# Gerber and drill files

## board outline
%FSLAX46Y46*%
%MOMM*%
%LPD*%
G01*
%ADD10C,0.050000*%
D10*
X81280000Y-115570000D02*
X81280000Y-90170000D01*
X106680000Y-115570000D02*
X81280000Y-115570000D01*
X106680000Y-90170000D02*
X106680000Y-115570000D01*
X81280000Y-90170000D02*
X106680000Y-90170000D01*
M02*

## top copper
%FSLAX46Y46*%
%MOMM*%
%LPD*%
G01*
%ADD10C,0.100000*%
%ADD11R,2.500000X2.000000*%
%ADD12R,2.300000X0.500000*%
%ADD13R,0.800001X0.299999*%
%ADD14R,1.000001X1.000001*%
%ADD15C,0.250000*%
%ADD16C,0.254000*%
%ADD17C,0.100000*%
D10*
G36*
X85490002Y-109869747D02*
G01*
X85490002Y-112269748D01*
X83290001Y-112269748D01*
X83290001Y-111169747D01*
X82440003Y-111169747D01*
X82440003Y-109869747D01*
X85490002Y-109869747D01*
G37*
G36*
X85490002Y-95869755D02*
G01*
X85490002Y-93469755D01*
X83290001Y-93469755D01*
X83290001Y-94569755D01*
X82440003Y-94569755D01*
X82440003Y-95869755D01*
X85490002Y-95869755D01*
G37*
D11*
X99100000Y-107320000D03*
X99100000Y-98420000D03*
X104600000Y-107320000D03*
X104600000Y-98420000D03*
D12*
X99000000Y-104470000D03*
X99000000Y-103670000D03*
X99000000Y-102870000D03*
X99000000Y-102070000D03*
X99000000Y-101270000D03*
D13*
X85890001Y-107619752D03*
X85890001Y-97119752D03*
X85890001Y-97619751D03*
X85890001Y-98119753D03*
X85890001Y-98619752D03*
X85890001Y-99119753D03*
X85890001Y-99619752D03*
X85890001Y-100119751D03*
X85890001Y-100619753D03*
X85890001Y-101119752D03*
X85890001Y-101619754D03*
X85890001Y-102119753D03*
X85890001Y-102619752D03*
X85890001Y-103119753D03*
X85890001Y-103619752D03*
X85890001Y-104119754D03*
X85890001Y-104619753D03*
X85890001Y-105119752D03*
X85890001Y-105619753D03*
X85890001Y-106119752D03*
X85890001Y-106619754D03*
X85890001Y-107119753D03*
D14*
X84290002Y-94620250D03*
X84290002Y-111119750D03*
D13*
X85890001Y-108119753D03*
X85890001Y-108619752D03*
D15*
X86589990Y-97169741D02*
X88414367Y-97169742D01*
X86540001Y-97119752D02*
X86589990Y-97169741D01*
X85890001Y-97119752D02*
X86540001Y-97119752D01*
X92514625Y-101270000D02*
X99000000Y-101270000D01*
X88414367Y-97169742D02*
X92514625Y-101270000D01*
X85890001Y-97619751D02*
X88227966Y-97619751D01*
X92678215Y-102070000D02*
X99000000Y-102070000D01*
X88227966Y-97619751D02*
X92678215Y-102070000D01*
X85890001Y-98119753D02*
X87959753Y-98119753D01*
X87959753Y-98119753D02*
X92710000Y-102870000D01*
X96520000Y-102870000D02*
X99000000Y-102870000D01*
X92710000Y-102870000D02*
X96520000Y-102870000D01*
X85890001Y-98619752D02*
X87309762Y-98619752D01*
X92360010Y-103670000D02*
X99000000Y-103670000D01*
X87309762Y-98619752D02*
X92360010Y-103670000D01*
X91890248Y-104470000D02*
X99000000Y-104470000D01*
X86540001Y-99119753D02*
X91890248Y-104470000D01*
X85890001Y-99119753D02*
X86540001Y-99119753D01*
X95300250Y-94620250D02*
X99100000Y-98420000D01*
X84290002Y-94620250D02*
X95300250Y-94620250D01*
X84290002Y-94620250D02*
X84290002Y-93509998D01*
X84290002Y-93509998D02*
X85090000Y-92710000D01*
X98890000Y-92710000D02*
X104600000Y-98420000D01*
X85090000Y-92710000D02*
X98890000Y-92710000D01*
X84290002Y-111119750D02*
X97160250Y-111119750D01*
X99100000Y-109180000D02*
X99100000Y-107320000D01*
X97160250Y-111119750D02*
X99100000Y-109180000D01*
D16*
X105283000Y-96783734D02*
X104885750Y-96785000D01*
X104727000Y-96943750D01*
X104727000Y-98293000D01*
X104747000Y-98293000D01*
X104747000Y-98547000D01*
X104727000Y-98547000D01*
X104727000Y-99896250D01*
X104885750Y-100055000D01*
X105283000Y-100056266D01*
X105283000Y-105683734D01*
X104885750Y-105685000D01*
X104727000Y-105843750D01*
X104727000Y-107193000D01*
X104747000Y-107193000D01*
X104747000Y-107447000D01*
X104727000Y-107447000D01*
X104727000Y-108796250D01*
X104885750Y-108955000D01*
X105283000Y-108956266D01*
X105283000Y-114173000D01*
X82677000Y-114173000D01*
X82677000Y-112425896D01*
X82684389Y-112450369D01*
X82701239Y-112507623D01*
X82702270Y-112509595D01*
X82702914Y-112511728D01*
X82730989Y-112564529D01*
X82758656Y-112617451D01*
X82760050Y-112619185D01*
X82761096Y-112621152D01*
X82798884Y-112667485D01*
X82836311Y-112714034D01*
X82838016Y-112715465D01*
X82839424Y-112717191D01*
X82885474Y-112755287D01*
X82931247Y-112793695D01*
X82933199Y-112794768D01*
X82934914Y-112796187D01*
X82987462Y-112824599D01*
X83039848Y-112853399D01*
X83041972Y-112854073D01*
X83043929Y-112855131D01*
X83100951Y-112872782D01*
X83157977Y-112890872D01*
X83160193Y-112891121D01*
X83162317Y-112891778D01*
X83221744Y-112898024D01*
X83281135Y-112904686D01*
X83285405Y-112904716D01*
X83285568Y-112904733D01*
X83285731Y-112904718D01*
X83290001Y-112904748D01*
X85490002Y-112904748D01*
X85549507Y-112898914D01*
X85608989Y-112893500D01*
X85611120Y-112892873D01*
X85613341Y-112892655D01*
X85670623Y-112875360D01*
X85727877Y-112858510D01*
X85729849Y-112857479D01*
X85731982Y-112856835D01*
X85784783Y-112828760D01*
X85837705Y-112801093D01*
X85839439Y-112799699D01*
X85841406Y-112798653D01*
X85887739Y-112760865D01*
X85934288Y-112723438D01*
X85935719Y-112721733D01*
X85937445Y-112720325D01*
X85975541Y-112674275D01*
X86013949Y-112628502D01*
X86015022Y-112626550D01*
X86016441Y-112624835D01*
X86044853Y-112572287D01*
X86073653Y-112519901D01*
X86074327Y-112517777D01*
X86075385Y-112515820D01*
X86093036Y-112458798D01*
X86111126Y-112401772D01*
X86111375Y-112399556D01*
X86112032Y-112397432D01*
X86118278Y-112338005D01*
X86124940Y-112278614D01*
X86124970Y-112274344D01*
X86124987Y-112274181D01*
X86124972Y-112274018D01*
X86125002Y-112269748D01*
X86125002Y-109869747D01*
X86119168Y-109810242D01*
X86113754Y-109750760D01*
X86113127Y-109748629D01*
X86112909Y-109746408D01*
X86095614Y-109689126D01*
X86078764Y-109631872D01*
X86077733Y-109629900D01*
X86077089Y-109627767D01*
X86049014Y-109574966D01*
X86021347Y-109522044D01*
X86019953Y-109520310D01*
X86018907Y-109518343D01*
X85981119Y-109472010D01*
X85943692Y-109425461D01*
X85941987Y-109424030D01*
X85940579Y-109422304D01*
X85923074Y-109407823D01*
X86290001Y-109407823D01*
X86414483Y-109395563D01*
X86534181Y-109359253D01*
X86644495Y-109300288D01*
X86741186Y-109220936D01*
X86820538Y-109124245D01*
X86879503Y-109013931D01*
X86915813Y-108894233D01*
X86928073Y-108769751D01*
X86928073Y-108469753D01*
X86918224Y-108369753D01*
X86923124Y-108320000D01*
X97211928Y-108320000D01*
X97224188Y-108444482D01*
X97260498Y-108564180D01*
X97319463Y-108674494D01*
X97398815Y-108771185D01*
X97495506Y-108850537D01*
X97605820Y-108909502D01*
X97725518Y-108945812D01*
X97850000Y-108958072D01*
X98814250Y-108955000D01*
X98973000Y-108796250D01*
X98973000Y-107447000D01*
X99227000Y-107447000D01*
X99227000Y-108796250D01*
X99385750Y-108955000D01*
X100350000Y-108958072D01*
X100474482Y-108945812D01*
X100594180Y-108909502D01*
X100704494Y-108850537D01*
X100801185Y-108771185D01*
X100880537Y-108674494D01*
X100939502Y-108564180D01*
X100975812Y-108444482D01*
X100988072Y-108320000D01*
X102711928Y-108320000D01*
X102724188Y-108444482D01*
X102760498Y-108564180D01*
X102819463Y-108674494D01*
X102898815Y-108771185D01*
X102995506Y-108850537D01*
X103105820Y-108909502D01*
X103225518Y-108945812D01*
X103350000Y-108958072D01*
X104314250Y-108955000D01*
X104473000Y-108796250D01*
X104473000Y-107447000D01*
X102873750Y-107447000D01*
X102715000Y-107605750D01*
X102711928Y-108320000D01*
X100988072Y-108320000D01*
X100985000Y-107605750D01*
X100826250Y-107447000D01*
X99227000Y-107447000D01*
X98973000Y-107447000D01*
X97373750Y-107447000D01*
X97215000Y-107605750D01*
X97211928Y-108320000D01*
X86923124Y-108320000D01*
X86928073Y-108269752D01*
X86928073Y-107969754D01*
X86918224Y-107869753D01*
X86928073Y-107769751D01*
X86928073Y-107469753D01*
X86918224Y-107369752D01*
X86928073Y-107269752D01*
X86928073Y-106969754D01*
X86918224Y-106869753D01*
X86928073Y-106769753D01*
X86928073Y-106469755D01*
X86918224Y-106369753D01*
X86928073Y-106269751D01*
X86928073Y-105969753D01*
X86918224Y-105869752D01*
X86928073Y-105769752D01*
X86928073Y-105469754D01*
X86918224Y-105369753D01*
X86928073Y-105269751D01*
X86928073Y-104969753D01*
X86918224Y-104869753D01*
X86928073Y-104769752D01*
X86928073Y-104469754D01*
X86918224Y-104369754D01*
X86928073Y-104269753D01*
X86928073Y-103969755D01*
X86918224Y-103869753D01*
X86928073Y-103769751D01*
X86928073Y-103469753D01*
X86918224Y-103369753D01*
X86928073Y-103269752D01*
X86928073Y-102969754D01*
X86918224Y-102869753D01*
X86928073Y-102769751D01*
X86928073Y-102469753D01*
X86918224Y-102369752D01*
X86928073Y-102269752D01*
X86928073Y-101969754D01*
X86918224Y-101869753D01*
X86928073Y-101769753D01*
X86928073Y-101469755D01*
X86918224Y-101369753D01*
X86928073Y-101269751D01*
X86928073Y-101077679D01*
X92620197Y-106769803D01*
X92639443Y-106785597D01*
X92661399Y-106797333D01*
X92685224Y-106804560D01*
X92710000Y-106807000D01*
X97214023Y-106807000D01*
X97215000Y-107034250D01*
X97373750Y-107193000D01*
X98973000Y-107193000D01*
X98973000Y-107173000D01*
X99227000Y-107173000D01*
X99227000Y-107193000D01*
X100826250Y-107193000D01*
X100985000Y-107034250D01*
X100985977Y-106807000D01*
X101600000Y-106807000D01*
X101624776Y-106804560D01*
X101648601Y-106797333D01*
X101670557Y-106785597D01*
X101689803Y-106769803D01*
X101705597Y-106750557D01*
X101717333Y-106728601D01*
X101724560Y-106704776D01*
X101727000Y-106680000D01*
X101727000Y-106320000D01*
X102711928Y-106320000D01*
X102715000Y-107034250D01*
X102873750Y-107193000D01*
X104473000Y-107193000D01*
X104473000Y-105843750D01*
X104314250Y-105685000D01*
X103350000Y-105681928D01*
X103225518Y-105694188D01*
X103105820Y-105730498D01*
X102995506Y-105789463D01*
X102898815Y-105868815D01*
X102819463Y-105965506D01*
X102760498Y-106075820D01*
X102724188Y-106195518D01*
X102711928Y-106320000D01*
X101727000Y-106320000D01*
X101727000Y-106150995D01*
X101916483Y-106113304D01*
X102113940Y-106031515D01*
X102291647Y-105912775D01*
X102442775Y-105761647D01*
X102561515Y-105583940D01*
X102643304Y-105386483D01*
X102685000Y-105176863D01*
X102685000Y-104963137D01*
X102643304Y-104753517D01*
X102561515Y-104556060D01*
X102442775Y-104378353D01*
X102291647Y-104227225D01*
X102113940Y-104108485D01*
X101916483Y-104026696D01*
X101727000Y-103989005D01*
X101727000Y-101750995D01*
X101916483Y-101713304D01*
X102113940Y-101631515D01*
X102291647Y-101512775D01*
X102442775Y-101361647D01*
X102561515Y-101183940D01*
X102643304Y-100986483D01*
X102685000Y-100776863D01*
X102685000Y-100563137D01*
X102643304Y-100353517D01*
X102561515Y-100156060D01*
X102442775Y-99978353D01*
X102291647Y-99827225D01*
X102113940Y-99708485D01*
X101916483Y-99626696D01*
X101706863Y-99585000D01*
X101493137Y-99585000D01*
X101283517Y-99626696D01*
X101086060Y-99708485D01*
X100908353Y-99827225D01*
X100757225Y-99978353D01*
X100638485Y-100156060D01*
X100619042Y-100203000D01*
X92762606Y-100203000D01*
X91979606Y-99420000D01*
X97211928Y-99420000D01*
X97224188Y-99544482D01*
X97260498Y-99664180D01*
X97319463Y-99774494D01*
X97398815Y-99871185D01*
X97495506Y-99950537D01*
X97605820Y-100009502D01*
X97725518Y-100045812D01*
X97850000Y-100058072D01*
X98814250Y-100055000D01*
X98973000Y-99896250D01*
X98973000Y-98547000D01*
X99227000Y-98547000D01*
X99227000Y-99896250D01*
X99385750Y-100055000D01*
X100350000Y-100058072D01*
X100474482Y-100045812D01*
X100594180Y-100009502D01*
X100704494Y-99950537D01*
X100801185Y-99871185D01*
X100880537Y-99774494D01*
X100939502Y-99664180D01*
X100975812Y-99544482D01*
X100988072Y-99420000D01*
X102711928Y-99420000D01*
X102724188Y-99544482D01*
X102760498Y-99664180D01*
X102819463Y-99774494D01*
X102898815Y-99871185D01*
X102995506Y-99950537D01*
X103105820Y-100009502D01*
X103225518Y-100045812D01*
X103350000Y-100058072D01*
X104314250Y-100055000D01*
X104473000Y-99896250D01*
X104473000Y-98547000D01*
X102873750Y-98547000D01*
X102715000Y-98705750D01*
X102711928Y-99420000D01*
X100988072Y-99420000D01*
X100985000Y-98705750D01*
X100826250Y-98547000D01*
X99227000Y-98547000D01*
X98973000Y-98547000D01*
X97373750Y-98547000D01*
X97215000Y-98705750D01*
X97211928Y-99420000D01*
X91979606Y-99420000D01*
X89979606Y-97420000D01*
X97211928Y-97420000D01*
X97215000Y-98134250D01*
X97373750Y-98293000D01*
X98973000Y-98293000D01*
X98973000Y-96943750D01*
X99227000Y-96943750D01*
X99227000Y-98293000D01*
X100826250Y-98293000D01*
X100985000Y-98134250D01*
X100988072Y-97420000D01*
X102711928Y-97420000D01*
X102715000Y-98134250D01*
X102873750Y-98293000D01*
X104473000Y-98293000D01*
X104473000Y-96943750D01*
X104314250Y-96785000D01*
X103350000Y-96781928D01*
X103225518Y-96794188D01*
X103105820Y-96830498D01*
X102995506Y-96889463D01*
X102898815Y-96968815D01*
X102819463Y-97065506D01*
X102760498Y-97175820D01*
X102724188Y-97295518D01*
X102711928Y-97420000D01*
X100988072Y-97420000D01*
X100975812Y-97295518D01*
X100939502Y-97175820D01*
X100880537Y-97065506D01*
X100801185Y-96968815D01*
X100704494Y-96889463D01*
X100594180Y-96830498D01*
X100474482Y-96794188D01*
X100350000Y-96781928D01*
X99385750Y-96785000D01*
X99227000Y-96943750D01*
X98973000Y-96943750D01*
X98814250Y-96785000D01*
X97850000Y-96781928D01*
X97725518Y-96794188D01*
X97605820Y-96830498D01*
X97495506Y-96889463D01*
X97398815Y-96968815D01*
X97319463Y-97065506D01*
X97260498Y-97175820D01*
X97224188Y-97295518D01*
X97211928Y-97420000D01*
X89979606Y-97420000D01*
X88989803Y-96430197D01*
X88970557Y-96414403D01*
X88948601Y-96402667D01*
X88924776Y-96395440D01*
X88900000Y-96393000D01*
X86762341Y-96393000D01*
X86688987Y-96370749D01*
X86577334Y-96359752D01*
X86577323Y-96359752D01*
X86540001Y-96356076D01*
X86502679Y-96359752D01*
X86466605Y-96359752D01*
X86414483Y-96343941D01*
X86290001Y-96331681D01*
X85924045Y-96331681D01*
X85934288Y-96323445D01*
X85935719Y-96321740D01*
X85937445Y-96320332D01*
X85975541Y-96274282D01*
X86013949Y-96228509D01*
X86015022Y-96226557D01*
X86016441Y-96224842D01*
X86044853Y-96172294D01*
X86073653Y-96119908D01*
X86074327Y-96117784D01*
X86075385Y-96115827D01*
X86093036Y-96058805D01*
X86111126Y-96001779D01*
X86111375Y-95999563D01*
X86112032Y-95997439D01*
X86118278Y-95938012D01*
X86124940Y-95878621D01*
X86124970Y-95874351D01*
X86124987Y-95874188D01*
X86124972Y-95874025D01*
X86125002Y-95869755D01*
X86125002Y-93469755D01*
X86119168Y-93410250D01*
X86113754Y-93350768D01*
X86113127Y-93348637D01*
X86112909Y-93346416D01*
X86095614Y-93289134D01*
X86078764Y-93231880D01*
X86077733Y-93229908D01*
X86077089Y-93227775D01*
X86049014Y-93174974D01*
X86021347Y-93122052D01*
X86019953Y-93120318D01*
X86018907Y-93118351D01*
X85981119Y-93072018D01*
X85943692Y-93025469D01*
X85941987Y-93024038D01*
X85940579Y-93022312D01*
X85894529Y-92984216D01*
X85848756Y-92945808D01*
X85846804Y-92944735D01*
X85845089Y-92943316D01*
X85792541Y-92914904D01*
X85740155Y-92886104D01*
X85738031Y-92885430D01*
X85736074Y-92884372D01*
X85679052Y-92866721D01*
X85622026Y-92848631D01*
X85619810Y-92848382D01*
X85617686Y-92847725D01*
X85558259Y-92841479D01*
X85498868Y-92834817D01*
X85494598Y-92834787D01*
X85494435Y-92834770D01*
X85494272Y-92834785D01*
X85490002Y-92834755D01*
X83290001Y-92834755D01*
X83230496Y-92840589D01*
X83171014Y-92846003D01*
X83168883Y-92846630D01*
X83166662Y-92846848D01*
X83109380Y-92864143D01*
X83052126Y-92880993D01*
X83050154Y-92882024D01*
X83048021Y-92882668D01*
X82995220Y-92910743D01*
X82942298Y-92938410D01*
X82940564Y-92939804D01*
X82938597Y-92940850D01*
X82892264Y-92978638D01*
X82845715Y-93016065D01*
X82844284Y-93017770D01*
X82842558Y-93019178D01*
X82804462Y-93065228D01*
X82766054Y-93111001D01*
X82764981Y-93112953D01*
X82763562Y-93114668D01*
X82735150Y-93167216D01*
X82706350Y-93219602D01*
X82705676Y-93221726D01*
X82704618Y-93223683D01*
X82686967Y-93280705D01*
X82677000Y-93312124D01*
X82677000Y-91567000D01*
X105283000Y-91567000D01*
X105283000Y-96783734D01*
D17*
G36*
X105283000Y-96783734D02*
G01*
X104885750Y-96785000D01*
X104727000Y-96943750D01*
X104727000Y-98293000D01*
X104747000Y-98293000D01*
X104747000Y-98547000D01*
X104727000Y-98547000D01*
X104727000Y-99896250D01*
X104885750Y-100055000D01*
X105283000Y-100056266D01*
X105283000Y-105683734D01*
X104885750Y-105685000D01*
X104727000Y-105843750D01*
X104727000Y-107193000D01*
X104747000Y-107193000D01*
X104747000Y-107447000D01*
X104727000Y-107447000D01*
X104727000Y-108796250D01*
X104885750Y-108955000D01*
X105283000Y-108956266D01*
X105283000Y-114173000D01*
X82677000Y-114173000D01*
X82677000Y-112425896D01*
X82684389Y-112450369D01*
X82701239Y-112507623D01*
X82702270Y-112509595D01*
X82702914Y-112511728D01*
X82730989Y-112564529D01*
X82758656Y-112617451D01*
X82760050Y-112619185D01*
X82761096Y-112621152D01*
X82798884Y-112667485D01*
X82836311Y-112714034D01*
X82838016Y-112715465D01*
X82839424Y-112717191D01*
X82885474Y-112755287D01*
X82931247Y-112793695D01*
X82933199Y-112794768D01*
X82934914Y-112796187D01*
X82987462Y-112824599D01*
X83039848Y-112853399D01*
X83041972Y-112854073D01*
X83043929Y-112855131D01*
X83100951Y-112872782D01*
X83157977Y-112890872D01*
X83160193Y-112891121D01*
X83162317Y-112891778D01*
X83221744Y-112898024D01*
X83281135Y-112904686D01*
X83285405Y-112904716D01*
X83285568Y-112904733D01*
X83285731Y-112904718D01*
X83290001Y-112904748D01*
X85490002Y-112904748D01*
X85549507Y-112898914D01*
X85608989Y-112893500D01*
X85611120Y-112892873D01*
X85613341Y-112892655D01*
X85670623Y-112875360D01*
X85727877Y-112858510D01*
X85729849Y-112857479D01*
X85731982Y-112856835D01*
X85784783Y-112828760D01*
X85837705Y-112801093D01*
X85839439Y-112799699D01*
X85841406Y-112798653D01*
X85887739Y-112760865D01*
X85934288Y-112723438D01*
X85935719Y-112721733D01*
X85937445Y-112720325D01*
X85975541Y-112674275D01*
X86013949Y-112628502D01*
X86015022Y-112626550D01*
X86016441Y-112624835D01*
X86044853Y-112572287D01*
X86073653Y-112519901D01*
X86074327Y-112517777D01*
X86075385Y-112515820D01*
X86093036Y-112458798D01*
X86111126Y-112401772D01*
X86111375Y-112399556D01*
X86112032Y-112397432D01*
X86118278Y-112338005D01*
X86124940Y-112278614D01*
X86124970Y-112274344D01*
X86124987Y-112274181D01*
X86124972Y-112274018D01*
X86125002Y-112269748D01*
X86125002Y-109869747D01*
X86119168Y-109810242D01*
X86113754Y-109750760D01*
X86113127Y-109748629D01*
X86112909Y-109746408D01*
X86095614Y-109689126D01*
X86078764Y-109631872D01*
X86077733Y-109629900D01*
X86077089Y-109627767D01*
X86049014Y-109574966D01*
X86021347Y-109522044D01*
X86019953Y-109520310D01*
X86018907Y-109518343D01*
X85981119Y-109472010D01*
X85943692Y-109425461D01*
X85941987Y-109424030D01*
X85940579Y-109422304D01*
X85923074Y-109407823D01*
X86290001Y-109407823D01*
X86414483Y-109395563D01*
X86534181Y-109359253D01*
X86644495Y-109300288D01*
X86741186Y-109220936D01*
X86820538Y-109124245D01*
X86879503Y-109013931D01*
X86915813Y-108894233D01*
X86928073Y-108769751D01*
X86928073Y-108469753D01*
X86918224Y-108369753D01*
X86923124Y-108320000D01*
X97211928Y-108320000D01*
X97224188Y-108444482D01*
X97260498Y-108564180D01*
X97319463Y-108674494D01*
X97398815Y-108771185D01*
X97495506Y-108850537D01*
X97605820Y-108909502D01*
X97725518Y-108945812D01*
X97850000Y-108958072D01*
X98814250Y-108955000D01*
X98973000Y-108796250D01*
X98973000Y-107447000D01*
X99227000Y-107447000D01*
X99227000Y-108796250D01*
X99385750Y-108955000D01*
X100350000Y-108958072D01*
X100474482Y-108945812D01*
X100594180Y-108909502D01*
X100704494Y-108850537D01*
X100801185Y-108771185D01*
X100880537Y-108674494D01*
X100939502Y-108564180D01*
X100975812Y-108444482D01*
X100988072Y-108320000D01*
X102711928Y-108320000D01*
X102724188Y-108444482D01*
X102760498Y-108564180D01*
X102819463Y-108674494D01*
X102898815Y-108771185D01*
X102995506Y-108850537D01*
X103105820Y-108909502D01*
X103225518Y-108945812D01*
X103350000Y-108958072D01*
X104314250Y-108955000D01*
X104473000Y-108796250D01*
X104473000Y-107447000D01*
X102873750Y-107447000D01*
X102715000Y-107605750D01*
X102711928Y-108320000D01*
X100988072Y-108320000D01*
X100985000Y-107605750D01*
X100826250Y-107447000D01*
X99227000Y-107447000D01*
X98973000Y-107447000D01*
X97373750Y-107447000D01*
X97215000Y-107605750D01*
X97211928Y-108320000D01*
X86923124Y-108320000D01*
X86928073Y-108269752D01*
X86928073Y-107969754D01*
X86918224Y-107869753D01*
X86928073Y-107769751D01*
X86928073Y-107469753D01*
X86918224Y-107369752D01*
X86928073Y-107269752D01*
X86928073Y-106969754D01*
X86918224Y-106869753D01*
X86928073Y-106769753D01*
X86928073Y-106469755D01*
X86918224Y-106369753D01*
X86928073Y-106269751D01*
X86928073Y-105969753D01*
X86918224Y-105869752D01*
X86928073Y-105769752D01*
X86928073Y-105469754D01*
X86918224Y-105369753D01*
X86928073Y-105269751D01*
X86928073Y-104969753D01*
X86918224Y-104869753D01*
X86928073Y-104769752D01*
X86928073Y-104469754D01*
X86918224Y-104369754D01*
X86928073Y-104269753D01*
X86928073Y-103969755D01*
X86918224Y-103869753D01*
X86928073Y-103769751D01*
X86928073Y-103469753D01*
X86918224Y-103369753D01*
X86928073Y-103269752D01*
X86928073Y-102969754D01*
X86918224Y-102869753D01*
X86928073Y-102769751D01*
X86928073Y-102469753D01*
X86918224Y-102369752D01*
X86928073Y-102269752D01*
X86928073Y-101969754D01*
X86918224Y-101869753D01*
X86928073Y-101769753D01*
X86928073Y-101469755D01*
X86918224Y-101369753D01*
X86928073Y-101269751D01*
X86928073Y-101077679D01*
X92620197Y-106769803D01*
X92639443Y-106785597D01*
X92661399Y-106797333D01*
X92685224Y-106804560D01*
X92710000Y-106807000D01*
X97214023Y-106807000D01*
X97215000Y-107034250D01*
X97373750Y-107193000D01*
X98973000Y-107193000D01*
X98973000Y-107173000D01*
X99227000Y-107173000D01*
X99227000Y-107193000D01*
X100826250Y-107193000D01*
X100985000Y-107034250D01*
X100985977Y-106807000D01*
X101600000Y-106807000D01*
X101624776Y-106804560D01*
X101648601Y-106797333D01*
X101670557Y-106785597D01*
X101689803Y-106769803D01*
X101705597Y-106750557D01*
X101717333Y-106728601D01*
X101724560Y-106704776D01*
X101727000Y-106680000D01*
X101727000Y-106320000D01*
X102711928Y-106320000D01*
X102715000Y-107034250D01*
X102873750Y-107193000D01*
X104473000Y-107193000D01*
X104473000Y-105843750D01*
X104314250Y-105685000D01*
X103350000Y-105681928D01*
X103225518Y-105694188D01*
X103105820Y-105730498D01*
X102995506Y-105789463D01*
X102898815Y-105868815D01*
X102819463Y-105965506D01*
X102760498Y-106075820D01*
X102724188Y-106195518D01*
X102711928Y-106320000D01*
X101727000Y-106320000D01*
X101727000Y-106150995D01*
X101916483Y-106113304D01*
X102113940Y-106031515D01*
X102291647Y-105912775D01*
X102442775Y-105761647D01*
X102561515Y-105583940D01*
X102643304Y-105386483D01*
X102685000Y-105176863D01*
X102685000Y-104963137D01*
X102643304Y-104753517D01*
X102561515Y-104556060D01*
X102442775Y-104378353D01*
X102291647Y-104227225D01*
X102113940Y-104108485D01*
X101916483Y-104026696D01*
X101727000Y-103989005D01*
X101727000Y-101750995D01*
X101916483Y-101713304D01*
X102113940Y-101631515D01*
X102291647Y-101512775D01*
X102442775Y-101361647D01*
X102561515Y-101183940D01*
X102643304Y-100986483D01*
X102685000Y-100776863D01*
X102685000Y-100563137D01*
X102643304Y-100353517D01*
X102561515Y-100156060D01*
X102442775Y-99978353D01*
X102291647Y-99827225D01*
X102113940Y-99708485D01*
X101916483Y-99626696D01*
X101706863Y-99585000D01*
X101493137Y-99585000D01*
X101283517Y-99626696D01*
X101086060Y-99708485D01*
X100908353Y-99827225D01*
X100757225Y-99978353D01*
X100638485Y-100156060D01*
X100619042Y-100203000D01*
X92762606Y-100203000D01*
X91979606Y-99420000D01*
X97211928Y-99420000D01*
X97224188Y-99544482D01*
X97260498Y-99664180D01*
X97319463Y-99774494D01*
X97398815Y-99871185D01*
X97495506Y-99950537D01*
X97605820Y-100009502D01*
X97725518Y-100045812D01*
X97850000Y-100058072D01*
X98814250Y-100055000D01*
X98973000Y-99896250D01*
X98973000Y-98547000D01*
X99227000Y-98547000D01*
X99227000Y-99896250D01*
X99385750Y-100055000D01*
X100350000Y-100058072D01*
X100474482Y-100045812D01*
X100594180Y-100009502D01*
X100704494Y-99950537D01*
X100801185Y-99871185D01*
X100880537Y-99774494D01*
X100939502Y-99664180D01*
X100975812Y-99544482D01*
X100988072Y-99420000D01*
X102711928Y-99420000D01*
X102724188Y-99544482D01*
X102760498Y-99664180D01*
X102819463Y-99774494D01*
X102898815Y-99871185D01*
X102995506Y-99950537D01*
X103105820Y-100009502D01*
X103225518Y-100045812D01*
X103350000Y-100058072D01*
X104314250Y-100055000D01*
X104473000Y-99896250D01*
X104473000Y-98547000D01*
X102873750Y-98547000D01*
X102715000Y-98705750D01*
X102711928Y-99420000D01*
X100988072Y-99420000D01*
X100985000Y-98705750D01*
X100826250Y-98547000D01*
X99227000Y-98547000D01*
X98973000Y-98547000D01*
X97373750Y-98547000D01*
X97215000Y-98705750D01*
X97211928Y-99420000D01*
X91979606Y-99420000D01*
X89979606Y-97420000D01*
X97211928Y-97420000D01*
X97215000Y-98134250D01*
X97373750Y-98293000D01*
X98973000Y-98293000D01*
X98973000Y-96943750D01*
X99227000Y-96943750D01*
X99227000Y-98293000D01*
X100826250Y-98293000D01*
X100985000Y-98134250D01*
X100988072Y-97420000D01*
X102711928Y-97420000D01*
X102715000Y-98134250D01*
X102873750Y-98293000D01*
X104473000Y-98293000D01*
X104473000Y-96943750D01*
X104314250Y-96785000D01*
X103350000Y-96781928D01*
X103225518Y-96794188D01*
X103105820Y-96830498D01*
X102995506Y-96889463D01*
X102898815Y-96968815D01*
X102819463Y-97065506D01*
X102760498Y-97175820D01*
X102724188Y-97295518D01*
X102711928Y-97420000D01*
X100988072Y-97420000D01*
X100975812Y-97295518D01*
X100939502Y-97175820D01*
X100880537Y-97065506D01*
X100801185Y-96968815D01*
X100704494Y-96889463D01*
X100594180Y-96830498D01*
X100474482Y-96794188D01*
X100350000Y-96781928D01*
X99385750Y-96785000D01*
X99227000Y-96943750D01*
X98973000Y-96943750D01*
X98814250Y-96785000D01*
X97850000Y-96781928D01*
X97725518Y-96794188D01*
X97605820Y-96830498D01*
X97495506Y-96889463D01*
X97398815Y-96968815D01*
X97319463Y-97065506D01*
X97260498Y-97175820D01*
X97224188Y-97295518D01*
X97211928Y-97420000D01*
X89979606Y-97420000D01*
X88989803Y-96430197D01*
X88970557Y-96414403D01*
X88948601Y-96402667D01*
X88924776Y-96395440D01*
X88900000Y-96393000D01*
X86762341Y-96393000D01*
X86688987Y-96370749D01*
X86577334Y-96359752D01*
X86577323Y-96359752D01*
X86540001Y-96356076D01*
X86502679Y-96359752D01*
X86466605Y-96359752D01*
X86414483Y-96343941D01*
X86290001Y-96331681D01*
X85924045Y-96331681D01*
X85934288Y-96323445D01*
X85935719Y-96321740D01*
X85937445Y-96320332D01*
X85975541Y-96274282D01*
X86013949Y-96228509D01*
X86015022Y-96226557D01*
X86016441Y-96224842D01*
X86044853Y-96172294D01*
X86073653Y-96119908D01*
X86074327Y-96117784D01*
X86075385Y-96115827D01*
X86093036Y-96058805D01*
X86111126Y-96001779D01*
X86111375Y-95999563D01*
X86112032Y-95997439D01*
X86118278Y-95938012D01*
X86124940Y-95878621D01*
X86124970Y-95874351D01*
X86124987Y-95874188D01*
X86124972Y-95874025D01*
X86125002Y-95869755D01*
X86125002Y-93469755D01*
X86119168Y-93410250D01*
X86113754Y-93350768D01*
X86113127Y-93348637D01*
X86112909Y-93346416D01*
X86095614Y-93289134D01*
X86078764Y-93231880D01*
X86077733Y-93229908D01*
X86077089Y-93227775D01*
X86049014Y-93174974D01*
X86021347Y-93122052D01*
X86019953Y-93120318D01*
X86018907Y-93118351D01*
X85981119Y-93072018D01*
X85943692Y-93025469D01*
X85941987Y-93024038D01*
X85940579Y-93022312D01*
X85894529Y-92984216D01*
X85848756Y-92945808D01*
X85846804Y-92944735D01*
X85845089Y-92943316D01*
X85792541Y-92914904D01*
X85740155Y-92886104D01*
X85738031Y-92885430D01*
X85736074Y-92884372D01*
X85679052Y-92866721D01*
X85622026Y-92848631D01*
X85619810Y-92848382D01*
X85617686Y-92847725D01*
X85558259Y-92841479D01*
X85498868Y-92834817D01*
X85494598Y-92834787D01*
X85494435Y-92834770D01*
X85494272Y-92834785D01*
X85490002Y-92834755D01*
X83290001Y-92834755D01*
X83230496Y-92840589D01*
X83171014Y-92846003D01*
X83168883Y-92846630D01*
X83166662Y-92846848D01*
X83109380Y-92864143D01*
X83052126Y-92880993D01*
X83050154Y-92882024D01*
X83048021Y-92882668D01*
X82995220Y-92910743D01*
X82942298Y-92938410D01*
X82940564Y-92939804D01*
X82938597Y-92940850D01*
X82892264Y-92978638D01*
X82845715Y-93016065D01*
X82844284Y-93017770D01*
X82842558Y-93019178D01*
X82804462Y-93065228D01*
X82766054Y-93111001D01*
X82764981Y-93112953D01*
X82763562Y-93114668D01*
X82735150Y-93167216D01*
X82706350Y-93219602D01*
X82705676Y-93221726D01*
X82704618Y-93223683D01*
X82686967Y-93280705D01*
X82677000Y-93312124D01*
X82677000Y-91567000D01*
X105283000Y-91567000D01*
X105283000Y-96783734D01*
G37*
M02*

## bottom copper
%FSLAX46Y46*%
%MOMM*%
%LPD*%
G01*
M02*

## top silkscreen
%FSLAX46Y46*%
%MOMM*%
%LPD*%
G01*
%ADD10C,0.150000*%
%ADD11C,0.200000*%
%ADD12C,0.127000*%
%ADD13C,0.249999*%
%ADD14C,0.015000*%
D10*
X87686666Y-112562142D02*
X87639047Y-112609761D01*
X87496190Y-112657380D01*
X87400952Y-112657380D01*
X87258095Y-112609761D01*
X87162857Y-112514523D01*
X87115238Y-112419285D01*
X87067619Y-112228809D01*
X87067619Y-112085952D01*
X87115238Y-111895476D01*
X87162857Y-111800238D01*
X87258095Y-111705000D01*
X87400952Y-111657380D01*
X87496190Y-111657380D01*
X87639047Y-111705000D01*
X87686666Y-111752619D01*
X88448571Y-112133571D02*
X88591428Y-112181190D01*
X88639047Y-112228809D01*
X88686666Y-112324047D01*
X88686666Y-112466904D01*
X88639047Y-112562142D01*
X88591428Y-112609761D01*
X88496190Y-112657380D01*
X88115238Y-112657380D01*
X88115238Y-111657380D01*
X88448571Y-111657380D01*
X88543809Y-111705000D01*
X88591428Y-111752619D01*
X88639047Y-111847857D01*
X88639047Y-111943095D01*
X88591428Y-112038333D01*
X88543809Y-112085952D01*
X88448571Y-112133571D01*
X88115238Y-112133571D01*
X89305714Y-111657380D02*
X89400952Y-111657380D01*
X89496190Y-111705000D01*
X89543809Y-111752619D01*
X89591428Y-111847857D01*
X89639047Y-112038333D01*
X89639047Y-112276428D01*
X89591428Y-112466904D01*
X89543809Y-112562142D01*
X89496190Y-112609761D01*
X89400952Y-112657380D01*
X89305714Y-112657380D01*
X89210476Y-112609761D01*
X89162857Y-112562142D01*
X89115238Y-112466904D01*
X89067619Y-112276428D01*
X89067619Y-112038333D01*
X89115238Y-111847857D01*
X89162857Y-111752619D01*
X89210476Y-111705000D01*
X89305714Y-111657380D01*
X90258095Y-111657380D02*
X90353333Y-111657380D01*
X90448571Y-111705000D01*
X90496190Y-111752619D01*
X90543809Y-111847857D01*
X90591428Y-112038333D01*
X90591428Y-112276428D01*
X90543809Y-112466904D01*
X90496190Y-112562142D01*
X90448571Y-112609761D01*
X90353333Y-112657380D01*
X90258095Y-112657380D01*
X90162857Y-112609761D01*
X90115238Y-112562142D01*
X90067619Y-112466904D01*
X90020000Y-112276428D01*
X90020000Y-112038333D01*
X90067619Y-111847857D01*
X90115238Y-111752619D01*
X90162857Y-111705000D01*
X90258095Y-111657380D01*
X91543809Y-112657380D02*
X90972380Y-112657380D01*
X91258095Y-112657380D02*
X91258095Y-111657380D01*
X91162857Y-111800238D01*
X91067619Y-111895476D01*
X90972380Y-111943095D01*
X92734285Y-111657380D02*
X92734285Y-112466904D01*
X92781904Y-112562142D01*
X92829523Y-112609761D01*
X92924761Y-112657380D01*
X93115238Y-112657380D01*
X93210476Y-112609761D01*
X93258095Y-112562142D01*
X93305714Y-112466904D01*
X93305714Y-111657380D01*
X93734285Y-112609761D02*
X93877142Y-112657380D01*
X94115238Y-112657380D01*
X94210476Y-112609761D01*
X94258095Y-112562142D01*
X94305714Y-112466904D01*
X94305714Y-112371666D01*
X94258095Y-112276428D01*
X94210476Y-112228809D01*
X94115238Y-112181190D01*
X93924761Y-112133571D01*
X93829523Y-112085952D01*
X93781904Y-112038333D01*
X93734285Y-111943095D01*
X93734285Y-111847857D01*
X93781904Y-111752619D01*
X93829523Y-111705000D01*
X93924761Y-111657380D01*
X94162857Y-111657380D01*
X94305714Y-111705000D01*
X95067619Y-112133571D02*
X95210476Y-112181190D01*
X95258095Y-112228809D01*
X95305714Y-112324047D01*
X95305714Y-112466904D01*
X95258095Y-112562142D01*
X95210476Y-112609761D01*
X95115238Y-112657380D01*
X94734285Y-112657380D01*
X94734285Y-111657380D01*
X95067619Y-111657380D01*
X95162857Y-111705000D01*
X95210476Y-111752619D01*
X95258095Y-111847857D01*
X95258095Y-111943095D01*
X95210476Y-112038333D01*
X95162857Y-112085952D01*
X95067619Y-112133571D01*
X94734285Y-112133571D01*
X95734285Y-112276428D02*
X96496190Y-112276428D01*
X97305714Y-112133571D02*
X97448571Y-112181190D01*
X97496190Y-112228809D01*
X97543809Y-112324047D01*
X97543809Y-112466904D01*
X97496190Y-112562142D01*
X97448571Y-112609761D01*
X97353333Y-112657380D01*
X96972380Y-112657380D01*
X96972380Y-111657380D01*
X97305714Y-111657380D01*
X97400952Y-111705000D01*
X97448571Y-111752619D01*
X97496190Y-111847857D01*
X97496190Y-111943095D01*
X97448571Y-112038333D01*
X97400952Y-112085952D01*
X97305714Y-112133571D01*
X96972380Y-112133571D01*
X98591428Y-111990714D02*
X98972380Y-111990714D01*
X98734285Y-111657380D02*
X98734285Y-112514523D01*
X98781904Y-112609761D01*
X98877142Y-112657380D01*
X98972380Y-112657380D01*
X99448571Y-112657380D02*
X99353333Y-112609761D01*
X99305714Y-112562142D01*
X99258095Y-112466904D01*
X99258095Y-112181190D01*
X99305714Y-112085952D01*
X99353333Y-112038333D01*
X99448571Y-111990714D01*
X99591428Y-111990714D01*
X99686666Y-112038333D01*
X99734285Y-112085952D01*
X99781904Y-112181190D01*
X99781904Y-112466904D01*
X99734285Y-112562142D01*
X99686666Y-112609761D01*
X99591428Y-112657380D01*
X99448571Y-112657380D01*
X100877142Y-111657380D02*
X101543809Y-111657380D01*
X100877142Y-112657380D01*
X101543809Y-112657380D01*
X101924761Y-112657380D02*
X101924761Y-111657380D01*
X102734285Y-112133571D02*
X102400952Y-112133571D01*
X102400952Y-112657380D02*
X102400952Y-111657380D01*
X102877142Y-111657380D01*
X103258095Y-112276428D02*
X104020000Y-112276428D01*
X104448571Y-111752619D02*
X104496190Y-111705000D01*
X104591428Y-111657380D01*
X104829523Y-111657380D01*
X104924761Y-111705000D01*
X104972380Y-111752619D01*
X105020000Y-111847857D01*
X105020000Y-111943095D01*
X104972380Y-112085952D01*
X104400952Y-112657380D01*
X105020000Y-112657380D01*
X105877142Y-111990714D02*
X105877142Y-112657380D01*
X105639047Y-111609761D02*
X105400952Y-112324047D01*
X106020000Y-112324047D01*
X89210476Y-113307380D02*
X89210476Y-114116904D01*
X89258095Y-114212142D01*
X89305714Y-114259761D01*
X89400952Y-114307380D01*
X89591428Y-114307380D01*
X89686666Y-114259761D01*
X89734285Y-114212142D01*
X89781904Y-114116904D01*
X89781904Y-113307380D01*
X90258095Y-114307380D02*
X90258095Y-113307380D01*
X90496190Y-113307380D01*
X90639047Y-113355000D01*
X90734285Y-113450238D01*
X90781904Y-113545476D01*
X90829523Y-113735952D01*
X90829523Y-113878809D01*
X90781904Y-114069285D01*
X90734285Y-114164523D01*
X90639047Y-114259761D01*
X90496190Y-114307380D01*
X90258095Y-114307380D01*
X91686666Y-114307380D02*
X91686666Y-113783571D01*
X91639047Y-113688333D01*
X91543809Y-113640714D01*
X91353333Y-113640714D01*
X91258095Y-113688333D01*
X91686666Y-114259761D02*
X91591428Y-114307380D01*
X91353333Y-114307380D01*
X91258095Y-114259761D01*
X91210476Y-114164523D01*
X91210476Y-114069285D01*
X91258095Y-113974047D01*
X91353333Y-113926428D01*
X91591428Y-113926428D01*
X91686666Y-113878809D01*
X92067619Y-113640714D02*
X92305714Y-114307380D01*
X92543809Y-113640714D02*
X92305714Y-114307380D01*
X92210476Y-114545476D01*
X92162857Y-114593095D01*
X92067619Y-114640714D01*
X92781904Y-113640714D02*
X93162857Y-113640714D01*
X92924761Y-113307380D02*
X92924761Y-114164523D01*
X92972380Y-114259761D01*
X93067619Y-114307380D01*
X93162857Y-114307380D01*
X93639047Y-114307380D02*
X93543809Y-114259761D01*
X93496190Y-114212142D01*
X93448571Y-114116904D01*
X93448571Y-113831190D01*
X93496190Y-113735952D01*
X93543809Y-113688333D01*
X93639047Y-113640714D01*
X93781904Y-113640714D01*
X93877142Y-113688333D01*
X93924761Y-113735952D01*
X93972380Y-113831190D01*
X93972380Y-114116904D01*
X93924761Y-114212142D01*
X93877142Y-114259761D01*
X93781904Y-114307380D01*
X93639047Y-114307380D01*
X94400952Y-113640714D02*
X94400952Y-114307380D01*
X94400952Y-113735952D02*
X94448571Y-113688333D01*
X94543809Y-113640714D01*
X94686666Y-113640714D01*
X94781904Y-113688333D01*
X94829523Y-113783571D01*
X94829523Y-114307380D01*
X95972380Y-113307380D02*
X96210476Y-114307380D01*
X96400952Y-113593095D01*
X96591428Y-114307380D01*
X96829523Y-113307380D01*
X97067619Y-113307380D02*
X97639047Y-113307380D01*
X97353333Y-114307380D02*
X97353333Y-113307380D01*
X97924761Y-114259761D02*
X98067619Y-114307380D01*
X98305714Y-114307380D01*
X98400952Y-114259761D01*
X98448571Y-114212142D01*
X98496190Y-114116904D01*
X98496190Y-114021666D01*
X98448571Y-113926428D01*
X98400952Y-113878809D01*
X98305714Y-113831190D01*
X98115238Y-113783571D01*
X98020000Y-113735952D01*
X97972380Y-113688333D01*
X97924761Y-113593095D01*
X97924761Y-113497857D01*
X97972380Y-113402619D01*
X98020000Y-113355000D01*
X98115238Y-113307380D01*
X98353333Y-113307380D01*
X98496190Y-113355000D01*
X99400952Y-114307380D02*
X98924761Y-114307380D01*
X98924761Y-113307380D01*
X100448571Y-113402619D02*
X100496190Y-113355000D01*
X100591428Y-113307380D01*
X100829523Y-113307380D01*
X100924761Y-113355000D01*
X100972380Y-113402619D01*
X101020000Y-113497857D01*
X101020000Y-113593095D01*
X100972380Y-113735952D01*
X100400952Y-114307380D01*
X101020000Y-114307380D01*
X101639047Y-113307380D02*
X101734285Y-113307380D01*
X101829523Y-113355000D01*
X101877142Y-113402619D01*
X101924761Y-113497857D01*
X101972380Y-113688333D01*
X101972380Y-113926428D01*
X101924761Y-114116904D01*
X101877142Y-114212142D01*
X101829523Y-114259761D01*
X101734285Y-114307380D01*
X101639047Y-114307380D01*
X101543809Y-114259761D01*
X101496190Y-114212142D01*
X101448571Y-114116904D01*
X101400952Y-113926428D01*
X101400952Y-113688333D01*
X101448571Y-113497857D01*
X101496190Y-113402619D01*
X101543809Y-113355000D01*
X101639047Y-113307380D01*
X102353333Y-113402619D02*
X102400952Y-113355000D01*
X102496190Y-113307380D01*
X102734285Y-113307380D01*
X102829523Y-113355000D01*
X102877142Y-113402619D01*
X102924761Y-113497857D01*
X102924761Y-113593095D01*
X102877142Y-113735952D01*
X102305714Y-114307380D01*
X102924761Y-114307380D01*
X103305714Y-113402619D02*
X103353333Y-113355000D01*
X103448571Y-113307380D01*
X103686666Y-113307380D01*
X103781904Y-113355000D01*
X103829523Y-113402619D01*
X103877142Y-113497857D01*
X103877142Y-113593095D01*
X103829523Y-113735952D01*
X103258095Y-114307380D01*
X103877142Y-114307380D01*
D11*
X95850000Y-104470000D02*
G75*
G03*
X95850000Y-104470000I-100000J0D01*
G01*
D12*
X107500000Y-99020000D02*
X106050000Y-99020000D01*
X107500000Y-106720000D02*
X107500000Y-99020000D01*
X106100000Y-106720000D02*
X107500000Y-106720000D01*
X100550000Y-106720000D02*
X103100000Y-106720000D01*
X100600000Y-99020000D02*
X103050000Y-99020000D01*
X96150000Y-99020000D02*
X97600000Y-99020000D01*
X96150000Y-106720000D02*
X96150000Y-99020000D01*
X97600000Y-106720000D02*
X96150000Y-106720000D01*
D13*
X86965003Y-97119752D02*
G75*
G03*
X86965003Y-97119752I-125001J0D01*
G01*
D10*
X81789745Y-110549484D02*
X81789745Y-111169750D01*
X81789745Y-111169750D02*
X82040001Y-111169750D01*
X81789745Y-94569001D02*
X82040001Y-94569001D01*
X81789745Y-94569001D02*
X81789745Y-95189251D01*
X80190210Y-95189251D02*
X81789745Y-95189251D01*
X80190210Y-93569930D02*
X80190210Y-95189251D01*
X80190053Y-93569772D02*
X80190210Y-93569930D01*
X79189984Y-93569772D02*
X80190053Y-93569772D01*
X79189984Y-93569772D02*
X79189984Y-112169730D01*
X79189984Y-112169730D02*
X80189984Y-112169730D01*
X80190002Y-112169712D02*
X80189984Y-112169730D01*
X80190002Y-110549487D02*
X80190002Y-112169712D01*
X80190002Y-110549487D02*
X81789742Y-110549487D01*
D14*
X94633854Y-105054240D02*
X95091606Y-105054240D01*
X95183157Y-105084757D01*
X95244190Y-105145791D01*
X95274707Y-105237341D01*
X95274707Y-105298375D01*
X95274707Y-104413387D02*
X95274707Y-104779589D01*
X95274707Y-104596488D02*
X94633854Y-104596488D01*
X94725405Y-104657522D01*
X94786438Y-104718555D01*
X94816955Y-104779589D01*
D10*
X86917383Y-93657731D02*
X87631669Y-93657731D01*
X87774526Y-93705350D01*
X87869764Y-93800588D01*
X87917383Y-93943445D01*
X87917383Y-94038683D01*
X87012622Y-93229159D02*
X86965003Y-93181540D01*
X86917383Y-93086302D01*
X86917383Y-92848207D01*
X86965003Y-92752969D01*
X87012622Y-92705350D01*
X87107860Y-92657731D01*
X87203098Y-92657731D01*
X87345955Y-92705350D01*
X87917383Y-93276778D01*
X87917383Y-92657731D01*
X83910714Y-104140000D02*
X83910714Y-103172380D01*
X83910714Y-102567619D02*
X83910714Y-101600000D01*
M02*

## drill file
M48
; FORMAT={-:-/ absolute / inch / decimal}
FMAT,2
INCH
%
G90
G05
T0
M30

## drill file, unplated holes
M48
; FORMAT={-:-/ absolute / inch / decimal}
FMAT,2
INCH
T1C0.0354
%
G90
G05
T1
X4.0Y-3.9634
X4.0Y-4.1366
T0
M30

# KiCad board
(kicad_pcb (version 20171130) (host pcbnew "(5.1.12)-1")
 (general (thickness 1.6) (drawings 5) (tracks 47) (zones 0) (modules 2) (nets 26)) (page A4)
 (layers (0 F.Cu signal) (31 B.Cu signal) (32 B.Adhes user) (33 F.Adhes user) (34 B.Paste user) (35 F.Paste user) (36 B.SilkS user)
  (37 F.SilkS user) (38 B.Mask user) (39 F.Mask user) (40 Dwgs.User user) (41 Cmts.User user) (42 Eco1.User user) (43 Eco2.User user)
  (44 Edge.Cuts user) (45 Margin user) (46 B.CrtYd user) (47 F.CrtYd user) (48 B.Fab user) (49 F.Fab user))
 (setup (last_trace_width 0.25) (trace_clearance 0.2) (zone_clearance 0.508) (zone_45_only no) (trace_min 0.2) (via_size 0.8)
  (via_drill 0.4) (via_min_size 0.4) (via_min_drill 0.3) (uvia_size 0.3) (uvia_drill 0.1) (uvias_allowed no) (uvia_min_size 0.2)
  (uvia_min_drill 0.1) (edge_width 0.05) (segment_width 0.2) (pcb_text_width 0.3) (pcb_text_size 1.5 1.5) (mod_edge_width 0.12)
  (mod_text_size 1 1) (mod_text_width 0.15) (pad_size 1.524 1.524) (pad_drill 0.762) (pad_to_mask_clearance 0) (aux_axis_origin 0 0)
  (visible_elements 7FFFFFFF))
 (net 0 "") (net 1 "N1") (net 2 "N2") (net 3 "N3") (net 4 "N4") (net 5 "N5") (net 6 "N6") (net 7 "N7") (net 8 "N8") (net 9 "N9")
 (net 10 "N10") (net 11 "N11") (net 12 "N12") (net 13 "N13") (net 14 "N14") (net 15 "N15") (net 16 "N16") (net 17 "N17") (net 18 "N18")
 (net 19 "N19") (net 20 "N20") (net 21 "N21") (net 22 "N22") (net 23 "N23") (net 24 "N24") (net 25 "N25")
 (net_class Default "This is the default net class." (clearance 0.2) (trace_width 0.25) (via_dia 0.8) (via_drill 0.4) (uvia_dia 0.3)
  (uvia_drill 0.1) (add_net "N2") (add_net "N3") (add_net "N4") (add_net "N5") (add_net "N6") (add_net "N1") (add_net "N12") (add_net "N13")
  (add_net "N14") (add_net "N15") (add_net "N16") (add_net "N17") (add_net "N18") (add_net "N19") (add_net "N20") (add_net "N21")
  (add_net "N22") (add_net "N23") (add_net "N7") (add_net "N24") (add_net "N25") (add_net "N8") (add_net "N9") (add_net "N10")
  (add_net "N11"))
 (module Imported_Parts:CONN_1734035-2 (layer F.Cu) (at 101.6 102.87 90)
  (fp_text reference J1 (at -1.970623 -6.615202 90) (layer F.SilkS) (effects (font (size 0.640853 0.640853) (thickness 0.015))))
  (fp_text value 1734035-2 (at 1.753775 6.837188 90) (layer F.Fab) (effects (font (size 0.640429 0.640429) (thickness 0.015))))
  (fp_line (start -3.85 -4) (end -3.85 -5.45) (layer F.SilkS) (width 0.127))
  (fp_line (start -3.85 -5.45) (end 3.85 -5.45) (layer F.SilkS) (width 0.127))
  (fp_line (start 3.85 -5.45) (end 3.85 -4) (layer F.SilkS) (width 0.127))
  (fp_line (start 3.85 -1) (end 3.85 1.45) (layer F.SilkS) (width 0.127))
  (fp_line (start -3.85 -1.05) (end -3.85 1.5) (layer F.SilkS) (width 0.127))
  (fp_line (start -3.85 4.5) (end -3.85 5.9) (layer F.SilkS) (width 0.127))
  (fp_line (start -3.85 5.9) (end 3.85 5.9) (layer F.SilkS) (width 0.127))
  (fp_line (start 3.85 5.9) (end 3.85 4.45) (layer F.SilkS) (width 0.127))
  (fp_circle (center -1.6 -5.85) (end -1.5 -5.85) (layer F.SilkS) (width 0.2))
  (pad S1 smd rect (at -4.45 -2.5 90) (size 2 2.5) (layers F.Cu F.Paste F.Mask) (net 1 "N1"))
  (pad S2 smd rect (at 4.45 -2.5 90) (size 2 2.5) (layers F.Cu F.Paste F.Mask) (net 1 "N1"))
  (pad S3 smd rect (at -4.45 3 90) (size 2 2.5) (layers F.Cu F.Paste F.Mask) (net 1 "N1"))
  (pad S4 smd rect (at 4.45 3 90) (size 2 2.5) (layers F.Cu F.Paste F.Mask) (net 1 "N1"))
  (pad None np_thru_hole circle (at -2.2 0 90) (size 0.9 0.9) (drill 0.9) (layers *.Cu *.Mask))
  (pad None np_thru_hole circle (at 2.2 0 90) (size 0.9 0.9) (drill 0.9) (layers *.Cu *.Mask))
  (pad 1 smd rect (at -1.6 -2.6 90) (size 0.5 2.3) (layers F.Cu F.Paste F.Mask) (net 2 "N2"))
  (pad 2 smd rect (at -0.8 -2.6 90) (size 0.5 2.3) (layers F.Cu F.Paste F.Mask) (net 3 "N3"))
  (pad 3 smd rect (at 0 -2.6 90) (size 0.5 2.3) (layers F.Cu F.Paste F.Mask) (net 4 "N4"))
  (pad 4 smd rect (at 0.8 -2.6 90) (size 0.5 2.3) (layers F.Cu F.Paste F.Mask) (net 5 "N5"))
  (pad 5 smd rect (at 1.6 -2.6 90) (size 0.5 2.3) (layers F.Cu F.Paste F.Mask) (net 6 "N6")))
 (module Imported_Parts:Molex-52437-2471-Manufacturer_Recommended (layer F.Cu) (at 85.09 102.87 270)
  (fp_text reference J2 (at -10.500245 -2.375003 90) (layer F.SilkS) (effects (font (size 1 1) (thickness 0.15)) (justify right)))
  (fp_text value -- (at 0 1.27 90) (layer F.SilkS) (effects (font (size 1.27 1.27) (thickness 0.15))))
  (fp_poly
   (pts (xy -7.000245 -0.400002) (xy -9.400245 -0.400002) (xy -9.400245 1.799999) (xy -8.300245 1.799999) (xy -8.300245 2.649997)
    (xy -7.000245 2.649997))
   (layer F.Cu) (width 0))
  (fp_poly
   (pts (xy 6.999747 -0.400002) (xy 9.399748 -0.400002) (xy 9.399748 1.799999) (xy 8.299747 1.799999) (xy 8.299747 2.649997)
    (xy 6.999747 2.649997))
   (layer F.Cu) (width 0))
  (fp_line (start 7.679487 4.899998) (end 7.679487 3.300258) (layer F.SilkS) (width 0.15))
  (fp_line (start 7.679487 4.899998) (end 9.299712 4.899998) (layer F.SilkS) (width 0.15))
  (fp_line (start 9.299712 4.899998) (end 9.29973 4.900016) (layer F.SilkS) (width 0.15))
  (fp_line (start 9.29973 5.900016) (end 9.29973 4.900016) (layer F.SilkS) (width 0.15))
  (fp_line (start -9.300228 5.900016) (end 9.29973 5.900016) (layer F.SilkS) (width 0.15))
  (fp_line (start -9.300228 5.900016) (end -9.300228 4.899947) (layer F.SilkS) (width 0.15))
  (fp_line (start -9.300228 4.899947) (end -9.30007 4.89979) (layer F.SilkS) (width 0.15))
  (fp_line (start -9.30007 4.89979) (end -7.680749 4.89979) (layer F.SilkS) (width 0.15))
  (fp_line (start -7.680749 4.89979) (end -7.680749 3.300255) (layer F.SilkS) (width 0.15))
  (fp_line (start -8.300999 3.300255) (end -7.680749 3.300255) (layer F.SilkS) (width 0.15))
  (fp_line (start -8.300999 3.300255) (end -8.300999 3.049999) (layer F.SilkS) (width 0.15))
  (fp_line (start 8.29975 3.300255) (end 8.29975 3.049999) (layer F.SilkS) (width 0.15))
  (fp_line (start 7.679484 3.300255) (end 8.29975 3.300255) (layer F.SilkS) (width 0.15))
  (fp_circle (center -5.750248 -1.750002) (end -5.625247 -1.750002) (layer F.SilkS) (width 0.249999))
  (pad 22 smd rect (at 4.749752 -0.800001 270) (size 0.299999 0.800001) (layers F.Cu F.Paste F.Mask) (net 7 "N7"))
  (pad 1 smd rect (at -5.750248 -0.800001 90) (size 0.299999 0.800001) (layers F.Cu F.Paste F.Mask) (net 6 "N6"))
  (pad 2 smd rect (at -5.250249 -0.800001 90) (size 0.299999 0.800001) (layers F.Cu F.Paste F.Mask) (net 5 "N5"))
  (pad 3 smd rect (at -4.750247 -0.800001 90) (size 0.299999 0.800001) (layers F.Cu F.Paste F.Mask) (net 4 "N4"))
  (pad 4 smd rect (at -4.250248 -0.800001 90) (size 0.299999 0.800001) (layers F.Cu F.Paste F.Mask) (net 3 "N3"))
  (pad 5 smd rect (at -3.750247 -0.800001 90) (size 0.299999 0.800001) (layers F.Cu F.Paste F.Mask) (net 2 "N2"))
  (pad 6 smd rect (at -3.250248 -0.800001 90) (size 0.299999 0.800001) (layers F.Cu F.Paste F.Mask) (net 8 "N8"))
  (pad 7 smd rect (at -2.750249 -0.800001 90) (size 0.299999 0.800001) (layers F.Cu F.Paste F.Mask) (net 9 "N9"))
  (pad 8 smd rect (at -2.250247 -0.800001 90) (size 0.299999 0.800001) (layers F.Cu F.Paste F.Mask) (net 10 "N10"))
  (pad 9 smd rect (at -1.750248 -0.800001 90) (size 0.299999 0.800001) (layers F.Cu F.Paste F.Mask) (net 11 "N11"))
  (pad 10 smd rect (at -1.250246 -0.800001 90) (size 0.299999 0.800001) (layers F.Cu F.Paste F.Mask) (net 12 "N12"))
  (pad 11 smd rect (at -0.750247 -0.800001 90) (size 0.299999 0.800001) (layers F.Cu F.Paste F.Mask) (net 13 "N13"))
  (pad 12 smd rect (at -0.250248 -0.800001 90) (size 0.299999 0.800001) (layers F.Cu F.Paste F.Mask) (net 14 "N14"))
  (pad 13 smd rect (at 0.249753 -0.800001 90) (size 0.299999 0.800001) (layers F.Cu F.Paste F.Mask) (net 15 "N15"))
  (pad 14 smd rect (at 0.749752 -0.800001 90) (size 0.299999 0.800001) (layers F.Cu F.Paste F.Mask) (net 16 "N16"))
  (pad 15 smd rect (at 1.249754 -0.800001 90) (size 0.299999 0.800001) (layers F.Cu F.Paste F.Mask) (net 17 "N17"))
  (pad 16 smd rect (at 1.749753 -0.800001 90) (size 0.299999 0.800001) (layers F.Cu F.Paste F.Mask) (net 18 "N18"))
  (pad 17 smd rect (at 2.249752 -0.800001 90) (size 0.299999 0.800001) (layers F.Cu F.Paste F.Mask) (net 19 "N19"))
  (pad 18 smd rect (at 2.749753 -0.800001 90) (size 0.299999 0.800001) (layers F.Cu F.Paste F.Mask) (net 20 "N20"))
  (pad 19 smd rect (at 3.249752 -0.800001 90) (size 0.299999 0.800001) (layers F.Cu F.Paste F.Mask) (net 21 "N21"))
  (pad 20 smd rect (at 3.749754 -0.800001 90) (size 0.299999 0.800001) (layers F.Cu F.Paste F.Mask) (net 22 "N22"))
  (pad 21 smd rect (at 4.249753 -0.800001 90) (size 0.299999 0.800001) (layers F.Cu F.Paste F.Mask) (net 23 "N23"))
  (pad MP1 smd rect (at -8.24975 0.799998 90) (size 1.000001 1.000001) (layers F.Cu F.Paste F.Mask) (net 1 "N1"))
  (pad MP2 smd rect (at 8.24975 0.799998 90) (size 1.000001 1.000001) (layers F.Cu F.Paste F.Mask) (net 1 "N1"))
  (pad 23 smd rect (at 5.249753 -0.800001 270) (size 0.299999 0.800001) (layers F.Cu F.Paste F.Mask) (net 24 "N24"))
  (pad 24 smd rect (at 5.749752 -0.800001 270) (size 0.299999 0.800001) (layers F.Cu F.Paste F.Mask) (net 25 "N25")))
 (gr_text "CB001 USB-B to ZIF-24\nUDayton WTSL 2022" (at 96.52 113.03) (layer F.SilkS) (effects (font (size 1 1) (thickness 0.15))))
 (gr_line (start 81.28 115.57) (end 81.28 90.17) (layer Edge.Cuts) (width 0.05))
 (gr_line (start 106.68 115.57) (end 81.28 115.57) (layer Edge.Cuts) (width 0.05))
 (gr_line (start 106.68 90.17) (end 106.68 115.57) (layer Edge.Cuts) (width 0.05))
 (gr_line (start 81.28 90.17) (end 106.68 90.17) (layer Edge.Cuts) (width 0.05))
 (segment (start 83.465001 110.359749) (end 83.530001 110.294749) (width 0.25) (layer F.Cu) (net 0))
 (segment (start 83.465001 111.760601) (end 83.465001 110.359749) (width 0.25) (layer F.Cu) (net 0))
 (segment (start 83.7184 112.014) (end 83.465001 111.760601) (width 0.25) (layer F.Cu) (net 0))
 (segment (start 83.7184 113.4872) (end 83.7184 112.014) (width 0.25) (layer F.Cu) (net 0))
 (segment (start 85.050004 110.294749) (end 85.424995 110.66974) (width 0.25) (layer F.Cu) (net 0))
 (segment (start 83.530001 110.294749) (end 85.050004 110.294749) (width 0.25) (layer F.Cu) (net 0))
 (segment (start 86.810009 113.073609) (end 85.30616 111.56976) (width 0.25) (layer F.Cu) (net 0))
 (segment (start 86.810009 113.622801) (end 86.810009 113.073609) (width 0.25) (layer F.Cu) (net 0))
 (segment (start 86.546401 113.886409) (end 86.810009 113.622801) (width 0.25) (layer F.Cu) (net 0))
 (segment (start 85.471658 113.886409) (end 86.546401 113.886409) (width 0.25) (layer F.Cu) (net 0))
 (segment (start 83.465001 111.879752) (end 85.471658 113.886409) (width 0.25) (layer F.Cu) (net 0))
 (segment (start 83.465001 110.359749) (end 83.465001 111.879752) (width 0.25) (layer F.Cu) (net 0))
 (segment (start 85.504349 110.294749) (end 85.87934 110.66974) (width 0.25) (layer F.Cu) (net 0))
 (segment (start 83.530001 110.294749) (end 85.504349 110.294749) (width 0.25) (layer F.Cu) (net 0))
 (segment (start 85.87934 110.66974) (end 86.868 110.66974) (width 0.25) (layer F.Cu) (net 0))
 (segment (start 86.868 110.66974) (end 85.17145 110.66974) (width 0.25) (layer F.Cu) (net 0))
 (segment (start 86.58999 97.169741) (end 88.414367 97.169742) (width 0.25) (layer F.Cu) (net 6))
 (segment (start 86.540001 97.119752) (end 86.58999 97.169741) (width 0.25) (layer F.Cu) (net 6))
 (segment (start 85.890001 97.119752) (end 86.540001 97.119752) (width 0.25) (layer F.Cu) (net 6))
 (segment (start 92.514625 101.27) (end 99 101.27) (width 0.25) (layer F.Cu) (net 6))
 (segment (start 88.414367 97.169742) (end 92.514625 101.27) (width 0.25) (layer F.Cu) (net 6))
 (segment (start 85.890001 97.619751) (end 88.227966 97.619751) (width 0.25) (layer F.Cu) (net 5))
 (segment (start 92.678215 102.07) (end 99 102.07) (width 0.25) (layer F.Cu) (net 5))
 (segment (start 88.227966 97.619751) (end 92.678215 102.07) (width 0.25) (layer F.Cu) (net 5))
 (segment (start 85.890001 98.119753) (end 87.959753 98.119753) (width 0.25) (layer F.Cu) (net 4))
 (segment (start 87.959753 98.119753) (end 92.71 102.87) (width 0.25) (layer F.Cu) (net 4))
 (segment (start 96.52 102.87) (end 99 102.87) (width 0.25) (layer F.Cu) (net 4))
 (segment (start 92.71 102.87) (end 96.52 102.87) (width 0.25) (layer F.Cu) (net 4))
 (segment (start 85.890001 98.619752) (end 87.309762 98.619752) (width 0.25) (layer F.Cu) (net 3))
 (segment (start 92.36001 103.67) (end 99 103.67) (width 0.25) (layer F.Cu) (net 3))
 (segment (start 87.309762 98.619752) (end 92.36001 103.67) (width 0.25) (layer F.Cu) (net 3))
 (segment (start 91.890248 104.47) (end 99 104.47) (width 0.25) (layer F.Cu) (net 2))
 (segment (start 86.540001 99.119753) (end 91.890248 104.47) (width 0.25) (layer F.Cu) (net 2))
 (segment (start 85.890001 99.119753) (end 86.540001 99.119753) (width 0.25) (layer F.Cu) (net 2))
 (segment (start 95.30025 94.62025) (end 99.1 98.42) (width 0.25) (layer F.Cu) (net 1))
 (segment (start 84.290002 94.62025) (end 95.30025 94.62025) (width 0.25) (layer F.Cu) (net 1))
 (segment (start 98.89 92.71) (end 104.6 98.42) (width 0.25) (layer F.Cu) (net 1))
 (segment (start 84.290002 111.11975) (end 97.16025 111.11975) (width 0.25) (layer F.Cu) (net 1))
 (segment (start 99.1 109.18) (end 99.1 107.32) (width 0.25) (layer F.Cu) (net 1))
 (segment (start 97.16025 111.11975) (end 99.1 109.18) (width 0.25) (layer F.Cu) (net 1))
 (segment (start 84.290002 111.366402) (end 84.290002 111.11975) (width 0.25) (layer F.Cu) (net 1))
 (segment (start 86.36 113.4364) (end 84.290002 111.366402) (width 0.25) (layer F.Cu) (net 1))
 (segment (start 84.29735 94.62025) (end 86.2076 92.71) (width 0.25) (layer F.Cu) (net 1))
 (segment (start 84.290002 94.62025) (end 84.29735 94.62025) (width 0.25) (layer F.Cu) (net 1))
 (segment (start 86.2076 92.71) (end 98.89 92.71) (width 0.25) (layer F.Cu) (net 1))
 (segment (start 85.122952 95.4532) (end 84.290002 94.62025) (width 0.25) (layer F.Cu) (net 1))
 (segment (start 88.0364 95.4532) (end 85.122952 95.4532) (width 0.25) (layer F.Cu) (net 1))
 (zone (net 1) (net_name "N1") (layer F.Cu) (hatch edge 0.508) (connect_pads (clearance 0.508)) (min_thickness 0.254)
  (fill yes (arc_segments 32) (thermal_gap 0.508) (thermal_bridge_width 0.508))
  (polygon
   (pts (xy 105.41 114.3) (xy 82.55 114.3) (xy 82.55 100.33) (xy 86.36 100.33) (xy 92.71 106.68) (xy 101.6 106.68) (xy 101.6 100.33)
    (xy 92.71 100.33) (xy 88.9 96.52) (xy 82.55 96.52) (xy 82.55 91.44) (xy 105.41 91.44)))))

